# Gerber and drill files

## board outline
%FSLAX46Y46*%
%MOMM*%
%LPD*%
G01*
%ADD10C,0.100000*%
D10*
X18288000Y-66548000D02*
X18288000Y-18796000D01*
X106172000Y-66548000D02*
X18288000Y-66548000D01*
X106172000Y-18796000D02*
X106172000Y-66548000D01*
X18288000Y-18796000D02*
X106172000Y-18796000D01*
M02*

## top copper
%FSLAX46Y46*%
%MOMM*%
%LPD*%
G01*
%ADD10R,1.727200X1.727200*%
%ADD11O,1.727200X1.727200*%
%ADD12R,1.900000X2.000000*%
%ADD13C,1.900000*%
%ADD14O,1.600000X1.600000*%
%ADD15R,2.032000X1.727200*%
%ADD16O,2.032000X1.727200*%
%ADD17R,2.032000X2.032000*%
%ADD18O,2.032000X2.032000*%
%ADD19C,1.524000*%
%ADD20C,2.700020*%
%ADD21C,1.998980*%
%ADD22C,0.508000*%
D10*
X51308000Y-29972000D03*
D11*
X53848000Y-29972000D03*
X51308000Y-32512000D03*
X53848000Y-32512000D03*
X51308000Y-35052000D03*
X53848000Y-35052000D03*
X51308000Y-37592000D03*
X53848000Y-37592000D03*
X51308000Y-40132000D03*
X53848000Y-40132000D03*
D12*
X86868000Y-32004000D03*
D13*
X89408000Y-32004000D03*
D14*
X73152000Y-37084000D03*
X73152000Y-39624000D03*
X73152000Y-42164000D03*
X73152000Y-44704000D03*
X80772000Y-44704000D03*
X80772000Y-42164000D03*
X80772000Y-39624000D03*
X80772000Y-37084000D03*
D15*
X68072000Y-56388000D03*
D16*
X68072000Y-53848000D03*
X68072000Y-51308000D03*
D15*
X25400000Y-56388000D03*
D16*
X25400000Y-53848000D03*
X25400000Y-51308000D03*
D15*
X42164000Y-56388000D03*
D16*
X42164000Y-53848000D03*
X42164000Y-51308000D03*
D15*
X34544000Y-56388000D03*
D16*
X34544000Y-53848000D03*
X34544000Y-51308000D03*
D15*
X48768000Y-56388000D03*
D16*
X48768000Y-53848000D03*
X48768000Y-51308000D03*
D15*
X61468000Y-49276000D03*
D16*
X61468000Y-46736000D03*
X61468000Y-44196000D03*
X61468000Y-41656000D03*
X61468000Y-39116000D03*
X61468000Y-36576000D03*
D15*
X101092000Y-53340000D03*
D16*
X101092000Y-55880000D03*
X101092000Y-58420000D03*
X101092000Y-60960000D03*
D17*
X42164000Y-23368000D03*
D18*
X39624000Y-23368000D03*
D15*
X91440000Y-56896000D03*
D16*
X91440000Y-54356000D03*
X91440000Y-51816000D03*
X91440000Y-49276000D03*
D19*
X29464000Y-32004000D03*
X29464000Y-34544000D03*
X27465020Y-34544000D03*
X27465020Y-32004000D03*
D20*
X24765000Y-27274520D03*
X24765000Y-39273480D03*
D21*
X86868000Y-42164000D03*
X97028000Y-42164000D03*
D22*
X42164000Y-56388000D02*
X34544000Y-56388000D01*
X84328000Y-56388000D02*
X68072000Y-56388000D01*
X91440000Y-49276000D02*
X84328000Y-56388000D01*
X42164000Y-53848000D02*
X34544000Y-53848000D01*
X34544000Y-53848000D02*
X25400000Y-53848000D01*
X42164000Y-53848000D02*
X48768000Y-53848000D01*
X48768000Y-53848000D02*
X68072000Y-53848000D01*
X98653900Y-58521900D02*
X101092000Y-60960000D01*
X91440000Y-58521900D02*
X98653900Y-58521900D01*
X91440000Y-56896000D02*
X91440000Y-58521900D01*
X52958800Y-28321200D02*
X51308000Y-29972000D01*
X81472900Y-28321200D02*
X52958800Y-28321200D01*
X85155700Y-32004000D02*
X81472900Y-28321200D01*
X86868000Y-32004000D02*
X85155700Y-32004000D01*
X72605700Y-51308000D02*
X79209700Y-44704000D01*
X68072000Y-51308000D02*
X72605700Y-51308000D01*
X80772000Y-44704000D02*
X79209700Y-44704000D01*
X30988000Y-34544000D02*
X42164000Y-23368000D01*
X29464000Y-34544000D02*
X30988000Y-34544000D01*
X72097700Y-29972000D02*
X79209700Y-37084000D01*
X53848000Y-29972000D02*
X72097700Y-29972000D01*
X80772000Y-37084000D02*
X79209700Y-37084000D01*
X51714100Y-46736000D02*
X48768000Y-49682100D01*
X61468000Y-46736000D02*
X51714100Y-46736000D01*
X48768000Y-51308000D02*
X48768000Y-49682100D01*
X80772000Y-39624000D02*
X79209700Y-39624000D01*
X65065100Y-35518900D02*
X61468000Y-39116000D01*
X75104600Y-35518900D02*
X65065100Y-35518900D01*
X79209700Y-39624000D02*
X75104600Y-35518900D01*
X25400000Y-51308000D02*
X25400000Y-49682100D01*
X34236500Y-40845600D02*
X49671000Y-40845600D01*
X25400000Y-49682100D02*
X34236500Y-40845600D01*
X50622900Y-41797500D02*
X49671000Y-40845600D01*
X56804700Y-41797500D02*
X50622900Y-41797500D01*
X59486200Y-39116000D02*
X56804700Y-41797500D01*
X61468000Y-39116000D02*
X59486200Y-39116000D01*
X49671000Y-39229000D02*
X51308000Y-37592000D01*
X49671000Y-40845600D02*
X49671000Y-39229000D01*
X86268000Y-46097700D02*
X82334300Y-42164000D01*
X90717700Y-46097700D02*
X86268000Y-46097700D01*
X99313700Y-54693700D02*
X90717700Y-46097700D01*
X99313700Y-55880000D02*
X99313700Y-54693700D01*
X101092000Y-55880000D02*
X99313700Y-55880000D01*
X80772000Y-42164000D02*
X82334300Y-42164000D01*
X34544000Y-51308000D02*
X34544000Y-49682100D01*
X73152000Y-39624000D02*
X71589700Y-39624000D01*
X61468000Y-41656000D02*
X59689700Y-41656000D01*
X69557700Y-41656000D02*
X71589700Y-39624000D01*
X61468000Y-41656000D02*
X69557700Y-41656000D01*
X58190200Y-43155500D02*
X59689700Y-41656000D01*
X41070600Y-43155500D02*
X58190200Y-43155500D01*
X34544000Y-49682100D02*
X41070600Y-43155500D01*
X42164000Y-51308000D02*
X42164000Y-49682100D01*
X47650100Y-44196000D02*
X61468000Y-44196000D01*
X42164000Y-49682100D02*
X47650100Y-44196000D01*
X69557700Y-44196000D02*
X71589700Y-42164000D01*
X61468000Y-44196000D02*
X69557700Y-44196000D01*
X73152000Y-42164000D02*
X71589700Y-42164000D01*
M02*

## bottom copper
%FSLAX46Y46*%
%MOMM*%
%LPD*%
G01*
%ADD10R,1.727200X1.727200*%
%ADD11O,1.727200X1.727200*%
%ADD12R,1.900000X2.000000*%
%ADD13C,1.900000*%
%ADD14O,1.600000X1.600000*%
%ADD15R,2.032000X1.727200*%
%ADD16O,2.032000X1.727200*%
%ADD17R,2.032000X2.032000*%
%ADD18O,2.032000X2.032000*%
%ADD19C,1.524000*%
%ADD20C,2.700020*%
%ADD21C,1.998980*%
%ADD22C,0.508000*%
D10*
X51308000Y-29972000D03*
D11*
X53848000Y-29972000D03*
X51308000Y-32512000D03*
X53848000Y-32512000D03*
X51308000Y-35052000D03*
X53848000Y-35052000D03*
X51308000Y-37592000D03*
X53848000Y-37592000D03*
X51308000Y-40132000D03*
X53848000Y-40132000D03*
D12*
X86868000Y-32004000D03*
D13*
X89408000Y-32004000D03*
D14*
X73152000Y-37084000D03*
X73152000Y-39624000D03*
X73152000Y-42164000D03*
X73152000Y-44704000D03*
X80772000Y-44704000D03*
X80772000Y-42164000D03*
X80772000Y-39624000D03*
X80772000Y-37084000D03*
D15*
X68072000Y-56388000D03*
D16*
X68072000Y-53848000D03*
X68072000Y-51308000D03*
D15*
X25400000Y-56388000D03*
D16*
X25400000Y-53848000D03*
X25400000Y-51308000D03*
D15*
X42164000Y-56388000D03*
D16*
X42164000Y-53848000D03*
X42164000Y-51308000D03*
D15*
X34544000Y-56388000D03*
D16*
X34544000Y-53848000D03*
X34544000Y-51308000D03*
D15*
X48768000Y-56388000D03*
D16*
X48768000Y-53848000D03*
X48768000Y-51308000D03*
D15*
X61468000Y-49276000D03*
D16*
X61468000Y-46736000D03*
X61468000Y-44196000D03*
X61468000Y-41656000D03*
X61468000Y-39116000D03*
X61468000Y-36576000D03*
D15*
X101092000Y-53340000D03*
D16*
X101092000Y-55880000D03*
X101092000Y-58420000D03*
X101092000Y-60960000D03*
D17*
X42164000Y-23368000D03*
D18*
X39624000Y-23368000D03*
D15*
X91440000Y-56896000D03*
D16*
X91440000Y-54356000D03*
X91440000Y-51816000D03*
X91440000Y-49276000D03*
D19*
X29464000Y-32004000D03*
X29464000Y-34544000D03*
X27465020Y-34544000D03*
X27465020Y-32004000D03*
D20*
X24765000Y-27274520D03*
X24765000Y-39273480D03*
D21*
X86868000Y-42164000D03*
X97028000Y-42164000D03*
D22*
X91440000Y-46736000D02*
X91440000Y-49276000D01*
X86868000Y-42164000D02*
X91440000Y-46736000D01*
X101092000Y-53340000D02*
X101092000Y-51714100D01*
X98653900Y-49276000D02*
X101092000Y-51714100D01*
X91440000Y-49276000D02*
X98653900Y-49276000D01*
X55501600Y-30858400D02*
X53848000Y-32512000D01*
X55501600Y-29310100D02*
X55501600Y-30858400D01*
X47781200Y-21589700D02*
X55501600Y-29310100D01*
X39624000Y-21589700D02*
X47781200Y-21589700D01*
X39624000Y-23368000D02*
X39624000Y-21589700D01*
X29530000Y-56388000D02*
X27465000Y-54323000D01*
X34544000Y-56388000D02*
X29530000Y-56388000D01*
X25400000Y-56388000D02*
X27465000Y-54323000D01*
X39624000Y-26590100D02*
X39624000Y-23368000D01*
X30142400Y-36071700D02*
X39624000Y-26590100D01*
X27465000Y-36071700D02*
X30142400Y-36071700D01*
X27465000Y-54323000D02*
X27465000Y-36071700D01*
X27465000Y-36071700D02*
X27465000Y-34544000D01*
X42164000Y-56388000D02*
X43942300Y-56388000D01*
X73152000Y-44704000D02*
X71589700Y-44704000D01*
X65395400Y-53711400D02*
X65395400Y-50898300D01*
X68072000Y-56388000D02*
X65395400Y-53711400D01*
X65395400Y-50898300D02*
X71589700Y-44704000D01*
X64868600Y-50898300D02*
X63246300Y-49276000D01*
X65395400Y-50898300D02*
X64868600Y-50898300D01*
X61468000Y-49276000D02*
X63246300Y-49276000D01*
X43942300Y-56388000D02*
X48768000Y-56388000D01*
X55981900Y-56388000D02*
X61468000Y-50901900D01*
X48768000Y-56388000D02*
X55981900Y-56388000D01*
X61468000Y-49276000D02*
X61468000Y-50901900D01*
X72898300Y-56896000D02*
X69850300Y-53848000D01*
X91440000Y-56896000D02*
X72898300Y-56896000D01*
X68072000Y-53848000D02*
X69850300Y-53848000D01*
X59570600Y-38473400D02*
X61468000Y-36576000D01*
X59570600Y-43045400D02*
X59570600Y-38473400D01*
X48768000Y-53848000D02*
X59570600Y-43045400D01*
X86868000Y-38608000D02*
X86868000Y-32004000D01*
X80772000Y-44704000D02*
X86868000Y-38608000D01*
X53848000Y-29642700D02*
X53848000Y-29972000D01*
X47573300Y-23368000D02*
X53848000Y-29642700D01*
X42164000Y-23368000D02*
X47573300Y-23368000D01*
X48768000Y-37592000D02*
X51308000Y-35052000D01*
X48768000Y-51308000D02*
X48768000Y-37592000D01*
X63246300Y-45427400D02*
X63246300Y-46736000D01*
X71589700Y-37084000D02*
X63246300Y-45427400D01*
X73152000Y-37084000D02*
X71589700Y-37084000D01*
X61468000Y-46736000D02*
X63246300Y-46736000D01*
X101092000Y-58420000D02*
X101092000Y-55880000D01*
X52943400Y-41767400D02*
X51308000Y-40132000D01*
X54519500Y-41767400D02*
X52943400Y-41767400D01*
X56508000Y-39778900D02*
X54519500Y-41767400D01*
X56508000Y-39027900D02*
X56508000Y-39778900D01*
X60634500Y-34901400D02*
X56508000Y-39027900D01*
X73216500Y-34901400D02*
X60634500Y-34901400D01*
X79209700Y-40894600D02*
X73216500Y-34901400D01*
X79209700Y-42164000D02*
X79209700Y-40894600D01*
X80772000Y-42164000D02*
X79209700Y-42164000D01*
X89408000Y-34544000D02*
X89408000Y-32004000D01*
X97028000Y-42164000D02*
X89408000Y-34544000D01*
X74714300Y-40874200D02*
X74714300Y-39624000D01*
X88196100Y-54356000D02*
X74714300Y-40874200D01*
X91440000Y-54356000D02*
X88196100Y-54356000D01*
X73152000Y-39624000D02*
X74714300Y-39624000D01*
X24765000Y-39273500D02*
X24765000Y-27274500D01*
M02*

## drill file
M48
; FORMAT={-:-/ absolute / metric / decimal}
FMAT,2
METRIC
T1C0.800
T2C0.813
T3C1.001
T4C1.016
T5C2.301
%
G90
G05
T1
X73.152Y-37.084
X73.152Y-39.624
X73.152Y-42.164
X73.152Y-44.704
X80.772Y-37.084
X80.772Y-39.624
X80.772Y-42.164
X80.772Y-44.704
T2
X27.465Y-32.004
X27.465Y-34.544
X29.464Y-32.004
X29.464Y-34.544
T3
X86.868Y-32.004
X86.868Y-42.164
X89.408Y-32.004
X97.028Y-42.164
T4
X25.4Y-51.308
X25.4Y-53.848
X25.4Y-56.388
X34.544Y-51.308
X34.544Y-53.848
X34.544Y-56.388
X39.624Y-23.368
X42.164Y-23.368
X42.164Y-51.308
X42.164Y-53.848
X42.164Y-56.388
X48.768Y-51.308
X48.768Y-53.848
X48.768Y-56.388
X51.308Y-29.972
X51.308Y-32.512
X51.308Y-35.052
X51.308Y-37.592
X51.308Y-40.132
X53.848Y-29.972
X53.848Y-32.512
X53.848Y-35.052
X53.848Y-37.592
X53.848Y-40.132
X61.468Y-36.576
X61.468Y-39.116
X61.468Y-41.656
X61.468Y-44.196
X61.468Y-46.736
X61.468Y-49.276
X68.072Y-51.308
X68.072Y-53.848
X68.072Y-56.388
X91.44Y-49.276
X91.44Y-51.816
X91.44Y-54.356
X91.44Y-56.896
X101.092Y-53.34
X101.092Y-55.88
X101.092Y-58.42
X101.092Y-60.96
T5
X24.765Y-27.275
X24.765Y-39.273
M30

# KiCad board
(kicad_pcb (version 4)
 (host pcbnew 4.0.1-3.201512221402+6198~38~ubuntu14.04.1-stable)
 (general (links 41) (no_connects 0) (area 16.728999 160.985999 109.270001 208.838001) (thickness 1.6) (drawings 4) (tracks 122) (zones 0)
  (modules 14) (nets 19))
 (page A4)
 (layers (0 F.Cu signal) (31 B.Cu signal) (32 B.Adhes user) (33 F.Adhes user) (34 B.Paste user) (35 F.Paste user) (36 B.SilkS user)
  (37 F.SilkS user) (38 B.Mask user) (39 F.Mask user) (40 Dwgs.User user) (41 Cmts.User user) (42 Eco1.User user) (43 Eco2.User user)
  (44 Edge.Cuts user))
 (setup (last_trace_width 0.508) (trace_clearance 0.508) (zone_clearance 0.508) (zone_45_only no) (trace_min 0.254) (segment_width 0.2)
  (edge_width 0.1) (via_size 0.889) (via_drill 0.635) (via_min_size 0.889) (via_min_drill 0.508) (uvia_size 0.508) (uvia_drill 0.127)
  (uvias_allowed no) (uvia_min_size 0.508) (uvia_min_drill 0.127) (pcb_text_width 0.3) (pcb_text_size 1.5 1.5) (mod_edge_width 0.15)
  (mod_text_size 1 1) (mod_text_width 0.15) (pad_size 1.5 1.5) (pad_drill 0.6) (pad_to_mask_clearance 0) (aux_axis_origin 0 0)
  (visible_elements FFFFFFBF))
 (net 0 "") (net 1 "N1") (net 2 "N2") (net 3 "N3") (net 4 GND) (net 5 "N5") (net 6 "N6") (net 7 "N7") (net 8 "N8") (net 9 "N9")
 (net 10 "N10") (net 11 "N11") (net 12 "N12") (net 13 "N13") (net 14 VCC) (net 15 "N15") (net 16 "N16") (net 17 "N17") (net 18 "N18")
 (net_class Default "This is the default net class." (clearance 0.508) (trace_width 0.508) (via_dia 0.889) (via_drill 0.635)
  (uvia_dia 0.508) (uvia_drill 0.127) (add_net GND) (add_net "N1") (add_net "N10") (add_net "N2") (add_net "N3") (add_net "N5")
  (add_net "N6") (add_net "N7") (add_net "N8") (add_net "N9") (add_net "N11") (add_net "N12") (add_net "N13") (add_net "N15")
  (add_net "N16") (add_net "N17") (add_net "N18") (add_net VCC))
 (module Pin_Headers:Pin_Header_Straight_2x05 (layer F.Cu) (at 51.308 29.972)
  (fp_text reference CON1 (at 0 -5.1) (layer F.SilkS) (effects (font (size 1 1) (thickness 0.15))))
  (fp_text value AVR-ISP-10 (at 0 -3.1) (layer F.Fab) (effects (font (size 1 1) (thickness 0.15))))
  (pad 1 thru_hole rect (at 0 0) (size 1.7272 1.7272) (drill 1.016) (layers *.Cu *.Mask F.SilkS) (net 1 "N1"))
  (pad 2 thru_hole oval (at 2.54 0) (size 1.7272 1.7272) (drill 1.016) (layers *.Cu *.Mask F.SilkS) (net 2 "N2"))
  (pad 3 thru_hole oval (at 0 2.54) (size 1.7272 1.7272) (drill 1.016) (layers *.Cu *.Mask F.SilkS) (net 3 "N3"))
  (pad 4 thru_hole oval (at 2.54 2.54) (size 1.7272 1.7272) (drill 1.016) (layers *.Cu *.Mask F.SilkS) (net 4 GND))
  (pad 5 thru_hole oval (at 0 5.08) (size 1.7272 1.7272) (drill 1.016) (layers *.Cu *.Mask F.SilkS) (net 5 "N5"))
  (pad 6 thru_hole oval (at 2.54 5.08) (size 1.7272 1.7272) (drill 1.016) (layers *.Cu *.Mask F.SilkS) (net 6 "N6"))
  (pad 7 thru_hole oval (at 0 7.62) (size 1.7272 1.7272) (drill 1.016) (layers *.Cu *.Mask F.SilkS) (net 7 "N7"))
  (pad 8 thru_hole oval (at 2.54 7.62) (size 1.7272 1.7272) (drill 1.016) (layers *.Cu *.Mask F.SilkS) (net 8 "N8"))
  (pad 9 thru_hole oval (at 0 10.16) (size 1.7272 1.7272) (drill 1.016) (layers *.Cu *.Mask F.SilkS) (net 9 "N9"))
  (pad 10 thru_hole oval (at 2.54 10.16) (size 1.7272 1.7272) (drill 1.016) (layers *.Cu *.Mask F.SilkS) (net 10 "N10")))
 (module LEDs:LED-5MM (layer F.Cu) (at 86.868 32.004)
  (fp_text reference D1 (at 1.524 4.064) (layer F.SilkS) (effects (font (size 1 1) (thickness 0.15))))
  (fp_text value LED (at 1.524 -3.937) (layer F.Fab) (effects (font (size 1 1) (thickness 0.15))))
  (pad 1 thru_hole rect (at 0 0 90) (size 2 1.9) (drill 1.00076) (layers *.Cu *.Mask F.SilkS) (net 1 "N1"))
  (pad 2 thru_hole circle (at 2.54 0) (size 1.9 1.9) (drill 1.00076) (layers *.Cu *.Mask F.SilkS) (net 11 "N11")))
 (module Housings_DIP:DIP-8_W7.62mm (layer F.Cu) (at 73.152 37.084)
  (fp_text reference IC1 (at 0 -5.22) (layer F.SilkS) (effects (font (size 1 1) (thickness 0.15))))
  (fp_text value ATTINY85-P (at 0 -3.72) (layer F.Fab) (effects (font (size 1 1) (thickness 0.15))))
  (pad 1 thru_hole oval (at 0 0) (size 1.6 1.6) (drill 0.8) (layers *.Cu *.Mask F.SilkS) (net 5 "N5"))
  (pad 2 thru_hole oval (at 0 2.54) (size 1.6 1.6) (drill 0.8) (layers *.Cu *.Mask F.SilkS) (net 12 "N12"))
  (pad 3 thru_hole oval (at 0 5.08) (size 1.6 1.6) (drill 0.8) (layers *.Cu *.Mask F.SilkS) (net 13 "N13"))
  (pad 4 thru_hole oval (at 0 7.62) (size 1.6 1.6) (drill 0.8) (layers *.Cu *.Mask F.SilkS) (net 4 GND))
  (pad 5 thru_hole oval (at 7.62 7.62) (size 1.6 1.6) (drill 0.8) (layers *.Cu *.Mask F.SilkS) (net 1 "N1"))
  (pad 6 thru_hole oval (at 7.62 5.08) (size 1.6 1.6) (drill 0.8) (layers *.Cu *.Mask F.SilkS) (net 9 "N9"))
  (pad 7 thru_hole oval (at 7.62 2.54) (size 1.6 1.6) (drill 0.8) (layers *.Cu *.Mask F.SilkS) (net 7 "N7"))
  (pad 8 thru_hole oval (at 7.62 0) (size 1.6 1.6) (drill 0.8) (layers *.Cu *.Mask F.SilkS) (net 2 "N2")))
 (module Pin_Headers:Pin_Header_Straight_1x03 (layer F.Cu) (at 68.072 56.388 180)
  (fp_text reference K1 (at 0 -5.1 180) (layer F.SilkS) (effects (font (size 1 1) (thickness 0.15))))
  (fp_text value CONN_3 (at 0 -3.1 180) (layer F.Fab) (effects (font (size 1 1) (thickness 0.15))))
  (pad 1 thru_hole rect (at 0 0 180) (size 2.032 1.7272) (drill 1.016) (layers *.Cu *.Mask F.SilkS) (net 4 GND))
  (pad 2 thru_hole oval (at 0 2.54 180) (size 2.032 1.7272) (drill 1.016) (layers *.Cu *.Mask F.SilkS) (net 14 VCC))
  (pad 3 thru_hole oval (at 0 5.08 180) (size 2.032 1.7272) (drill 1.016) (layers *.Cu *.Mask F.SilkS) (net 1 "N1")))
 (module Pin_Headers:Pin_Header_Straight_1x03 (layer F.Cu) (at 25.4 56.388 180)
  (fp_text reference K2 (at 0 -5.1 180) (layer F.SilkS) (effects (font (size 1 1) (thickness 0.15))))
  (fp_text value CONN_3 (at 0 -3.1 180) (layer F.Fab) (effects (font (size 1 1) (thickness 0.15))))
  (pad 1 thru_hole rect (at 0 0 180) (size 2.032 1.7272) (drill 1.016) (layers *.Cu *.Mask F.SilkS) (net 4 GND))
  (pad 2 thru_hole oval (at 0 2.54 180) (size 2.032 1.7272) (drill 1.016) (layers *.Cu *.Mask F.SilkS) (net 14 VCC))
  (pad 3 thru_hole oval (at 0 5.08 180) (size 2.032 1.7272) (drill 1.016) (layers *.Cu *.Mask F.SilkS) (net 7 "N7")))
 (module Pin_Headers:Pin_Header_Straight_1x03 (layer F.Cu) (at 42.164 56.388 180)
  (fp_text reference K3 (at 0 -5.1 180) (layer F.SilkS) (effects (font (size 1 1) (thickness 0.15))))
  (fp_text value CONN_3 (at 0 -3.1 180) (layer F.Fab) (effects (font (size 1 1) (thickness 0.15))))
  (pad 1 thru_hole rect (at 0 0 180) (size 2.032 1.7272) (drill 1.016) (layers *.Cu *.Mask F.SilkS) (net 4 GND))
  (pad 2 thru_hole oval (at 0 2.54 180) (size 2.032 1.7272) (drill 1.016) (layers *.Cu *.Mask F.SilkS) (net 14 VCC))
  (pad 3 thru_hole oval (at 0 5.08 180) (size 2.032 1.7272) (drill 1.016) (layers *.Cu *.Mask F.SilkS) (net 13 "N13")))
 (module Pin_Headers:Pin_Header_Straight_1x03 (layer F.Cu) (at 34.544 56.388 180)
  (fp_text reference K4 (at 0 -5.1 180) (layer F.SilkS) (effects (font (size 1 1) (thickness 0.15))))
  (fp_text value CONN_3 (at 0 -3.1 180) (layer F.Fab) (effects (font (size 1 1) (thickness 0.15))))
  (pad 1 thru_hole rect (at 0 0 180) (size 2.032 1.7272) (drill 1.016) (layers *.Cu *.Mask F.SilkS) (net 4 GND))
  (pad 2 thru_hole oval (at 0 2.54 180) (size 2.032 1.7272) (drill 1.016) (layers *.Cu *.Mask F.SilkS) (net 14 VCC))
  (pad 3 thru_hole oval (at 0 5.08 180) (size 2.032 1.7272) (drill 1.016) (layers *.Cu *.Mask F.SilkS) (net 12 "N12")))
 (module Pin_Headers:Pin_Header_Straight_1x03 (layer F.Cu) (at 48.768 56.388 180)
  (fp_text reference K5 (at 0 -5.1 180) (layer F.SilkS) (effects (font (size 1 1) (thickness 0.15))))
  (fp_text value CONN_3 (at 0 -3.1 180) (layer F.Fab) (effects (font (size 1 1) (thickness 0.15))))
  (pad 1 thru_hole rect (at 0 0 180) (size 2.032 1.7272) (drill 1.016) (layers *.Cu *.Mask F.SilkS) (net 4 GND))
  (pad 2 thru_hole oval (at 0 2.54 180) (size 2.032 1.7272) (drill 1.016) (layers *.Cu *.Mask F.SilkS) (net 14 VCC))
  (pad 3 thru_hole oval (at 0 5.08 180) (size 2.032 1.7272) (drill 1.016) (layers *.Cu *.Mask F.SilkS) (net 5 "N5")))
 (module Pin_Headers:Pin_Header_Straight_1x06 (layer F.Cu) (at 61.468 49.276 180)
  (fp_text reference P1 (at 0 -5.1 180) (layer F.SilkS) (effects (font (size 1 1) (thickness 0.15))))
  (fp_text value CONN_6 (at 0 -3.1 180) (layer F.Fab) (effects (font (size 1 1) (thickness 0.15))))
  (pad 1 thru_hole rect (at 0 0 180) (size 2.032 1.7272) (drill 1.016) (layers *.Cu *.Mask F.SilkS) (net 4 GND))
  (pad 2 thru_hole oval (at 0 2.54 180) (size 2.032 1.7272) (drill 1.016) (layers *.Cu *.Mask F.SilkS) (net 5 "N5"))
  (pad 3 thru_hole oval (at 0 5.08 180) (size 2.032 1.7272) (drill 1.016) (layers *.Cu *.Mask F.SilkS) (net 13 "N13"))
  (pad 4 thru_hole oval (at 0 7.62 180) (size 2.032 1.7272) (drill 1.016) (layers *.Cu *.Mask F.SilkS) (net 12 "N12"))
  (pad 5 thru_hole oval (at 0 10.16 180) (size 2.032 1.7272) (drill 1.016) (layers *.Cu *.Mask F.SilkS) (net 7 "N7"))
  (pad 6 thru_hole oval (at 0 12.7 180) (size 2.032 1.7272) (drill 1.016) (layers *.Cu *.Mask F.SilkS) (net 14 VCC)))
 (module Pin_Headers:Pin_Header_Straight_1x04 (layer F.Cu) (at 101.092 53.34)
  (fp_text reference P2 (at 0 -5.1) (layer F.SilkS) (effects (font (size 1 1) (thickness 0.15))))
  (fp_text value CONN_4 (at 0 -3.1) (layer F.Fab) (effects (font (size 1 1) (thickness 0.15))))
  (pad 1 thru_hole rect (at 0 0) (size 2.032 1.7272) (drill 1.016) (layers *.Cu *.Mask F.SilkS) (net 4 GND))
  (pad 2 thru_hole oval (at 0 2.54) (size 2.032 1.7272) (drill 1.016) (layers *.Cu *.Mask F.SilkS) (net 9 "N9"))
  (pad 3 thru_hole oval (at 0 5.08) (size 2.032 1.7272) (drill 1.016) (layers *.Cu *.Mask F.SilkS) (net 9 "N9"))
  (pad 4 thru_hole oval (at 0 7.62) (size 2.032 1.7272) (drill 1.016) (layers *.Cu *.Mask F.SilkS) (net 14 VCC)))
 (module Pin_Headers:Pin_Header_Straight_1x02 (layer F.Cu) (at 42.164 23.368 270)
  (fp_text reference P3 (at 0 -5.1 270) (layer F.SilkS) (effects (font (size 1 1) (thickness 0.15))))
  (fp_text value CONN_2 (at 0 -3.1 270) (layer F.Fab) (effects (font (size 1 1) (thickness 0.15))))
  (pad 1 thru_hole rect (at 0 0 270) (size 2.032 2.032) (drill 1.016) (layers *.Cu *.Mask F.SilkS) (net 2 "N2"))
  (pad 2 thru_hole oval (at 0 2.54 270) (size 2.032 2.032) (drill 1.016) (layers *.Cu *.Mask F.SilkS) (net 4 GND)))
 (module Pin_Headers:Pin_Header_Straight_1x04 (layer F.Cu) (at 91.44 56.896 180)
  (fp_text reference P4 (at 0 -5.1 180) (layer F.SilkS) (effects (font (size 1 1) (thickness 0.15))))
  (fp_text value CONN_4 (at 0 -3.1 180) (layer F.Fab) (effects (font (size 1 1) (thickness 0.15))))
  (pad 1 thru_hole rect (at 0 0 180) (size 2.032 1.7272) (drill 1.016) (layers *.Cu *.Mask F.SilkS) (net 14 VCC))
  (pad 2 thru_hole oval (at 0 2.54 180) (size 2.032 1.7272) (drill 1.016) (layers *.Cu *.Mask F.SilkS) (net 12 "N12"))
  (pad 3 thru_hole oval (at 0 5.08 180) (size 2.032 1.7272) (drill 1.016) (layers *.Cu *.Mask F.SilkS) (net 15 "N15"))
  (pad 4 thru_hole oval (at 0 7.62 180) (size 2.032 1.7272) (drill 1.016) (layers *.Cu *.Mask F.SilkS) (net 4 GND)))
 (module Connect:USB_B (layer F.Cu) (at 29.464 34.544 180)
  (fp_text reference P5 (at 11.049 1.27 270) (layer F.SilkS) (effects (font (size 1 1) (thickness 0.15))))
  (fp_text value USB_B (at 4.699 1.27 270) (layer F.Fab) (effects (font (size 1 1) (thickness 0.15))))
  (pad 2 thru_hole circle (at 0 2.54 90) (size 1.524 1.524) (drill 0.8128) (layers *.Cu *.Mask F.SilkS) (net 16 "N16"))
  (pad 1 thru_hole circle (at 0 0 90) (size 1.524 1.524) (drill 0.8128) (layers *.Cu *.Mask F.SilkS) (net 2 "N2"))
  (pad 4 thru_hole circle (at 1.99898 0 90) (size 1.524 1.524) (drill 0.8128) (layers *.Cu *.Mask F.SilkS) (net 4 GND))
  (pad 3 thru_hole circle (at 1.99898 2.54 90) (size 1.524 1.524) (drill 0.8128) (layers *.Cu *.Mask F.SilkS) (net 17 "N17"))
  (pad 5 thru_hole circle (at 4.699 7.26948 90) (size 2.70002 2.70002) (drill 2.30124) (layers *.Cu *.Mask F.SilkS) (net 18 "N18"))
  (pad 5 thru_hole circle (at 4.699 -4.72948 90) (size 2.70002 2.70002) (drill 2.30124) (layers *.Cu *.Mask F.SilkS) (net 18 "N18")))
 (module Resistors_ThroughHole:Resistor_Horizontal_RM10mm (layer F.Cu) (at 91.948 42.164)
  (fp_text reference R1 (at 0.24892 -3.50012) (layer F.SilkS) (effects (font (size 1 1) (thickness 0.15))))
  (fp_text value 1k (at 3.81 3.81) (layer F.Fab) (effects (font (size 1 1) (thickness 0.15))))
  (pad 1 thru_hole circle (at -5.08 0) (size 1.99898 1.99898) (drill 1.00076) (layers *.Cu *.SilkS *.Mask) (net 4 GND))
  (pad 2 thru_hole circle (at 5.08 0) (size 1.99898 1.99898) (drill 1.00076) (layers *.Cu *.SilkS *.Mask) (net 11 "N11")))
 (gr_line (start 18.288 66.548) (end 18.288 18.796) (angle 90) (layer Edge.Cuts) (width 0.1))
 (gr_line (start 106.172 66.548) (end 18.288 66.548) (angle 90) (layer Edge.Cuts) (width 0.1))
 (gr_line (start 106.172 18.796) (end 106.172 66.548) (angle 90) (layer Edge.Cuts) (width 0.1))
 (gr_line (start 18.288 18.796) (end 106.172 18.796) (angle 90) (layer Edge.Cuts) (width 0.1))
 (segment (start 91.44 46.736) (end 91.44 49.276) (width 0.508) (layer B.Cu) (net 4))
 (segment (start 86.868 42.164) (end 91.44 46.736) (width 0.508) (layer B.Cu) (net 4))
 (segment (start 101.092 53.34) (end 101.092 51.7141) (width 0.508) (layer B.Cu) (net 4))
 (segment (start 98.6539 49.276) (end 101.092 51.7141) (width 0.508) (layer B.Cu) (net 4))
 (segment (start 91.44 49.276) (end 98.6539 49.276) (width 0.508) (layer B.Cu) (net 4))
 (segment (start 42.164 56.388) (end 34.544 56.388) (width 0.508) (layer F.Cu) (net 4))
 (segment (start 55.5016 30.8584) (end 53.848 32.512) (width 0.508) (layer B.Cu) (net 4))
 (segment (start 55.5016 29.3101) (end 55.5016 30.8584) (width 0.508) (layer B.Cu) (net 4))
 (segment (start 47.7812 21.5897) (end 55.5016 29.3101) (width 0.508) (layer B.Cu) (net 4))
 (segment (start 39.624 21.5897) (end 47.7812 21.5897) (width 0.508) (layer B.Cu) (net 4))
 (segment (start 39.624 23.368) (end 39.624 21.5897) (width 0.508) (layer B.Cu) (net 4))
 (segment (start 29.53 56.388) (end 27.465 54.323) (width 0.508) (layer B.Cu) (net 4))
 (segment (start 34.544 56.388) (end 29.53 56.388) (width 0.508) (layer B.Cu) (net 4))
 (segment (start 25.4 56.388) (end 27.465 54.323) (width 0.508) (layer B.Cu) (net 4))
 (segment (start 39.624 26.5901) (end 39.624 23.368) (width 0.508) (layer B.Cu) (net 4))
 (segment (start 30.1424 36.0717) (end 39.624 26.5901) (width 0.508) (layer B.Cu) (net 4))
 (segment (start 27.465 36.0717) (end 30.1424 36.0717) (width 0.508) (layer B.Cu) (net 4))
 (segment (start 27.465 54.323) (end 27.465 36.0717) (width 0.508) (layer B.Cu) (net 4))
 (segment (start 27.465 36.0717) (end 27.465 34.544) (width 0.508) (layer B.Cu) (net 4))
 (segment (start 42.164 56.388) (end 43.9423 56.388) (width 0.508) (layer B.Cu) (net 4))
 (segment (start 73.152 44.704) (end 71.5897 44.704) (width 0.508) (layer B.Cu) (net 4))
 (segment (start 65.3954 53.7114) (end 65.3954 50.8983) (width 0.508) (layer B.Cu) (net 4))
 (segment (start 68.072 56.388) (end 65.3954 53.7114) (width 0.508) (layer B.Cu) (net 4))
 (segment (start 65.3954 50.8983) (end 71.5897 44.704) (width 0.508) (layer B.Cu) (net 4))
 (segment (start 64.8686 50.8983) (end 63.2463 49.276) (width 0.508) (layer B.Cu) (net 4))
 (segment (start 65.3954 50.8983) (end 64.8686 50.8983) (width 0.508) (layer B.Cu) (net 4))
 (segment (start 61.468 49.276) (end 63.2463 49.276) (width 0.508) (layer B.Cu) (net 4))
 (segment (start 43.9423 56.388) (end 48.768 56.388) (width 0.508) (layer B.Cu) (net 4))
 (segment (start 55.9819 56.388) (end 61.468 50.9019) (width 0.508) (layer B.Cu) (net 4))
 (segment (start 48.768 56.388) (end 55.9819 56.388) (width 0.508) (layer B.Cu) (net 4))
 (segment (start 61.468 49.276) (end 61.468 50.9019) (width 0.508) (layer B.Cu) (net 4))
 (segment (start 84.328 56.388) (end 68.072 56.388) (width 0.508) (layer F.Cu) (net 4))
 (segment (start 91.44 49.276) (end 84.328 56.388) (width 0.508) (layer F.Cu) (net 4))
 (segment (start 42.164 53.848) (end 34.544 53.848) (width 0.508) (layer F.Cu) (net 14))
 (segment (start 34.544 53.848) (end 25.4 53.848) (width 0.508) (layer F.Cu) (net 14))
 (segment (start 42.164 53.848) (end 48.768 53.848) (width 0.508) (layer F.Cu) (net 14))
 (segment (start 48.768 53.848) (end 68.072 53.848) (width 0.508) (layer F.Cu) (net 14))
 (segment (start 98.6539 58.5219) (end 101.092 60.96) (width 0.508) (layer F.Cu) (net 14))
 (segment (start 91.44 58.5219) (end 98.6539 58.5219) (width 0.508) (layer F.Cu) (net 14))
 (segment (start 91.44 56.896) (end 91.44 58.5219) (width 0.508) (layer F.Cu) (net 14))
 (segment (start 72.8983 56.896) (end 69.8503 53.848) (width 0.508) (layer B.Cu) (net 14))
 (segment (start 91.44 56.896) (end 72.8983 56.896) (width 0.508) (layer B.Cu) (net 14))
 (segment (start 68.072 53.848) (end 69.8503 53.848) (width 0.508) (layer B.Cu) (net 14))
 (segment (start 59.5706 38.4734) (end 61.468 36.576) (width 0.508) (layer B.Cu) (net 14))
 (segment (start 59.5706 43.0454) (end 59.5706 38.4734) (width 0.508) (layer B.Cu) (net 14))
 (segment (start 48.768 53.848) (end 59.5706 43.0454) (width 0.508) (layer B.Cu) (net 14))
 (segment (start 86.868 38.608) (end 86.868 32.004) (width 0.508) (layer B.Cu) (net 1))
 (segment (start 80.772 44.704) (end 86.868 38.608) (width 0.508) (layer B.Cu) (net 1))
 (segment (start 52.9588 28.3212) (end 51.308 29.972) (width 0.508) (layer F.Cu) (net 1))
 (segment (start 81.4729 28.3212) (end 52.9588 28.3212) (width 0.508) (layer F.Cu) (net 1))
 (segment (start 85.1557 32.004) (end 81.4729 28.3212) (width 0.508) (layer F.Cu) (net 1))
 (segment (start 86.868 32.004) (end 85.1557 32.004) (width 0.508) (layer F.Cu) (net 1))
 (segment (start 72.6057 51.308) (end 79.2097 44.704) (width 0.508) (layer F.Cu) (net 1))
 (segment (start 68.072 51.308) (end 72.6057 51.308) (width 0.508) (layer F.Cu) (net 1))
 (segment (start 80.772 44.704) (end 79.2097 44.704) (width 0.508) (layer F.Cu) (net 1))
 (segment (start 30.988 34.544) (end 42.164 23.368) (width 0.508) (layer F.Cu) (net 2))
 (segment (start 29.464 34.544) (end 30.988 34.544) (width 0.508) (layer F.Cu) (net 2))
 (segment (start 72.0977 29.972) (end 79.2097 37.084) (width 0.508) (layer F.Cu) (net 2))
 (segment (start 53.848 29.972) (end 72.0977 29.972) (width 0.508) (layer F.Cu) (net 2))
 (segment (start 80.772 37.084) (end 79.2097 37.084) (width 0.508) (layer F.Cu) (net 2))
 (segment (start 53.848 29.6427) (end 53.848 29.972) (width 0.508) (layer B.Cu) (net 2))
 (segment (start 47.5733 23.368) (end 53.848 29.6427) (width 0.508) (layer B.Cu) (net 2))
 (segment (start 42.164 23.368) (end 47.5733 23.368) (width 0.508) (layer B.Cu) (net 2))
 (segment (start 51.7141 46.736) (end 48.768 49.6821) (width 0.508) (layer F.Cu) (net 5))
 (segment (start 61.468 46.736) (end 51.7141 46.736) (width 0.508) (layer F.Cu) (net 5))
 (segment (start 48.768 51.308) (end 48.768 49.6821) (width 0.508) (layer F.Cu) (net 5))
 (segment (start 48.768 37.592) (end 51.308 35.052) (width 0.508) (layer B.Cu) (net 5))
 (segment (start 48.768 51.308) (end 48.768 37.592) (width 0.508) (layer B.Cu) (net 5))
 (segment (start 63.2463 45.4274) (end 63.2463 46.736) (width 0.508) (layer B.Cu) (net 5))
 (segment (start 71.5897 37.084) (end 63.2463 45.4274) (width 0.508) (layer B.Cu) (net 5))
 (segment (start 73.152 37.084) (end 71.5897 37.084) (width 0.508) (layer B.Cu) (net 5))
 (segment (start 61.468 46.736) (end 63.2463 46.736) (width 0.508) (layer B.Cu) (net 5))
 (segment (start 80.772 39.624) (end 79.2097 39.624) (width 0.508) (layer F.Cu) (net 7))
 (segment (start 65.0651 35.5189) (end 61.468 39.116) (width 0.508) (layer F.Cu) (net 7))
 (segment (start 75.1046 35.5189) (end 65.0651 35.5189) (width 0.508) (layer F.Cu) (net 7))
 (segment (start 79.2097 39.624) (end 75.1046 35.5189) (width 0.508) (layer F.Cu) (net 7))
 (segment (start 25.4 51.308) (end 25.4 49.6821) (width 0.508) (layer F.Cu) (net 7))
 (segment (start 34.2365 40.8456) (end 49.671 40.8456) (width 0.508) (layer F.Cu) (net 7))
 (segment (start 25.4 49.6821) (end 34.2365 40.8456) (width 0.508) (layer F.Cu) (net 7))
 (segment (start 50.6229 41.7975) (end 49.671 40.8456) (width 0.508) (layer F.Cu) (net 7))
 (segment (start 56.8047 41.7975) (end 50.6229 41.7975) (width 0.508) (layer F.Cu) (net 7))
 (segment (start 59.4862 39.116) (end 56.8047 41.7975) (width 0.508) (layer F.Cu) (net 7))
 (segment (start 61.468 39.116) (end 59.4862 39.116) (width 0.508) (layer F.Cu) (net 7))
 (segment (start 49.671 39.229) (end 51.308 37.592) (width 0.508) (layer F.Cu) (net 7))
 (segment (start 49.671 40.8456) (end 49.671 39.229) (width 0.508) (layer F.Cu) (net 7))
 (segment (start 101.092 58.42) (end 101.092 55.88) (width 0.508) (layer B.Cu) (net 9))
 (segment (start 86.268 46.0977) (end 82.3343 42.164) (width 0.508) (layer F.Cu) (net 9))
 (segment (start 90.7177 46.0977) (end 86.268 46.0977) (width 0.508) (layer F.Cu) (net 9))
 (segment (start 99.3137 54.6937) (end 90.7177 46.0977) (width 0.508) (layer F.Cu) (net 9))
 (segment (start 99.3137 55.88) (end 99.3137 54.6937) (width 0.508) (layer F.Cu) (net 9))
 (segment (start 101.092 55.88) (end 99.3137 55.88) (width 0.508) (layer F.Cu) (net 9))
 (segment (start 80.772 42.164) (end 82.3343 42.164) (width 0.508) (layer F.Cu) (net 9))
 (segment (start 52.9434 41.7674) (end 51.308 40.132) (width 0.508) (layer B.Cu) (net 9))
 (segment (start 54.5195 41.7674) (end 52.9434 41.7674) (width 0.508) (layer B.Cu) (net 9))
 (segment (start 56.508 39.7789) (end 54.5195 41.7674) (width 0.508) (layer B.Cu) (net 9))
 (segment (start 56.508 39.0279) (end 56.508 39.7789) (width 0.508) (layer B.Cu) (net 9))
 (segment (start 60.6345 34.9014) (end 56.508 39.0279) (width 0.508) (layer B.Cu) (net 9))
 (segment (start 73.2165 34.9014) (end 60.6345 34.9014) (width 0.508) (layer B.Cu) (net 9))
 (segment (start 79.2097 40.8946) (end 73.2165 34.9014) (width 0.508) (layer B.Cu) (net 9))
 (segment (start 79.2097 42.164) (end 79.2097 40.8946) (width 0.508) (layer B.Cu) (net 9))
 (segment (start 80.772 42.164) (end 79.2097 42.164) (width 0.508) (layer B.Cu) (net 9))
 (segment (start 89.408 34.544) (end 89.408 32.004) (width 0.508) (layer B.Cu) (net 11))
 (segment (start 97.028 42.164) (end 89.408 34.544) (width 0.508) (layer B.Cu) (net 11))
 (segment (start 34.544 51.308) (end 34.544 49.6821) (width 0.508) (layer F.Cu) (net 12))
 (segment (start 73.152 39.624) (end 71.5897 39.624) (width 0.508) (layer F.Cu) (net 12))
 (segment (start 61.468 41.656) (end 59.6897 41.656) (width 0.508) (layer F.Cu) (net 12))
 (segment (start 69.5577 41.656) (end 71.5897 39.624) (width 0.508) (layer F.Cu) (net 12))
 (segment (start 61.468 41.656) (end 69.5577 41.656) (width 0.508) (layer F.Cu) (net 12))
 (segment (start 58.1902 43.1555) (end 59.6897 41.656) (width 0.508) (layer F.Cu) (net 12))
 (segment (start 41.0706 43.1555) (end 58.1902 43.1555) (width 0.508) (layer F.Cu) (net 12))
 (segment (start 34.544 49.6821) (end 41.0706 43.1555) (width 0.508) (layer F.Cu) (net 12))
 (segment (start 74.7143 40.8742) (end 74.7143 39.624) (width 0.508) (layer B.Cu) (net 12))
 (segment (start 88.1961 54.356) (end 74.7143 40.8742) (width 0.508) (layer B.Cu) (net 12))
 (segment (start 91.44 54.356) (end 88.1961 54.356) (width 0.508) (layer B.Cu) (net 12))
 (segment (start 73.152 39.624) (end 74.7143 39.624) (width 0.508) (layer B.Cu) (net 12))
 (segment (start 42.164 51.308) (end 42.164 49.6821) (width 0.508) (layer F.Cu) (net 13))
 (segment (start 47.6501 44.196) (end 61.468 44.196) (width 0.508) (layer F.Cu) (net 13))
 (segment (start 42.164 49.6821) (end 47.6501 44.196) (width 0.508) (layer F.Cu) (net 13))
 (segment (start 69.5577 44.196) (end 71.5897 42.164) (width 0.508) (layer F.Cu) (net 13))
 (segment (start 61.468 44.196) (end 69.5577 44.196) (width 0.508) (layer F.Cu) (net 13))
 (segment (start 73.152 42.164) (end 71.5897 42.164) (width 0.508) (layer F.Cu) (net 13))
 (segment (start 24.765 39.2735) (end 24.765 27.2745) (width 0.508) (layer B.Cu) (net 18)))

